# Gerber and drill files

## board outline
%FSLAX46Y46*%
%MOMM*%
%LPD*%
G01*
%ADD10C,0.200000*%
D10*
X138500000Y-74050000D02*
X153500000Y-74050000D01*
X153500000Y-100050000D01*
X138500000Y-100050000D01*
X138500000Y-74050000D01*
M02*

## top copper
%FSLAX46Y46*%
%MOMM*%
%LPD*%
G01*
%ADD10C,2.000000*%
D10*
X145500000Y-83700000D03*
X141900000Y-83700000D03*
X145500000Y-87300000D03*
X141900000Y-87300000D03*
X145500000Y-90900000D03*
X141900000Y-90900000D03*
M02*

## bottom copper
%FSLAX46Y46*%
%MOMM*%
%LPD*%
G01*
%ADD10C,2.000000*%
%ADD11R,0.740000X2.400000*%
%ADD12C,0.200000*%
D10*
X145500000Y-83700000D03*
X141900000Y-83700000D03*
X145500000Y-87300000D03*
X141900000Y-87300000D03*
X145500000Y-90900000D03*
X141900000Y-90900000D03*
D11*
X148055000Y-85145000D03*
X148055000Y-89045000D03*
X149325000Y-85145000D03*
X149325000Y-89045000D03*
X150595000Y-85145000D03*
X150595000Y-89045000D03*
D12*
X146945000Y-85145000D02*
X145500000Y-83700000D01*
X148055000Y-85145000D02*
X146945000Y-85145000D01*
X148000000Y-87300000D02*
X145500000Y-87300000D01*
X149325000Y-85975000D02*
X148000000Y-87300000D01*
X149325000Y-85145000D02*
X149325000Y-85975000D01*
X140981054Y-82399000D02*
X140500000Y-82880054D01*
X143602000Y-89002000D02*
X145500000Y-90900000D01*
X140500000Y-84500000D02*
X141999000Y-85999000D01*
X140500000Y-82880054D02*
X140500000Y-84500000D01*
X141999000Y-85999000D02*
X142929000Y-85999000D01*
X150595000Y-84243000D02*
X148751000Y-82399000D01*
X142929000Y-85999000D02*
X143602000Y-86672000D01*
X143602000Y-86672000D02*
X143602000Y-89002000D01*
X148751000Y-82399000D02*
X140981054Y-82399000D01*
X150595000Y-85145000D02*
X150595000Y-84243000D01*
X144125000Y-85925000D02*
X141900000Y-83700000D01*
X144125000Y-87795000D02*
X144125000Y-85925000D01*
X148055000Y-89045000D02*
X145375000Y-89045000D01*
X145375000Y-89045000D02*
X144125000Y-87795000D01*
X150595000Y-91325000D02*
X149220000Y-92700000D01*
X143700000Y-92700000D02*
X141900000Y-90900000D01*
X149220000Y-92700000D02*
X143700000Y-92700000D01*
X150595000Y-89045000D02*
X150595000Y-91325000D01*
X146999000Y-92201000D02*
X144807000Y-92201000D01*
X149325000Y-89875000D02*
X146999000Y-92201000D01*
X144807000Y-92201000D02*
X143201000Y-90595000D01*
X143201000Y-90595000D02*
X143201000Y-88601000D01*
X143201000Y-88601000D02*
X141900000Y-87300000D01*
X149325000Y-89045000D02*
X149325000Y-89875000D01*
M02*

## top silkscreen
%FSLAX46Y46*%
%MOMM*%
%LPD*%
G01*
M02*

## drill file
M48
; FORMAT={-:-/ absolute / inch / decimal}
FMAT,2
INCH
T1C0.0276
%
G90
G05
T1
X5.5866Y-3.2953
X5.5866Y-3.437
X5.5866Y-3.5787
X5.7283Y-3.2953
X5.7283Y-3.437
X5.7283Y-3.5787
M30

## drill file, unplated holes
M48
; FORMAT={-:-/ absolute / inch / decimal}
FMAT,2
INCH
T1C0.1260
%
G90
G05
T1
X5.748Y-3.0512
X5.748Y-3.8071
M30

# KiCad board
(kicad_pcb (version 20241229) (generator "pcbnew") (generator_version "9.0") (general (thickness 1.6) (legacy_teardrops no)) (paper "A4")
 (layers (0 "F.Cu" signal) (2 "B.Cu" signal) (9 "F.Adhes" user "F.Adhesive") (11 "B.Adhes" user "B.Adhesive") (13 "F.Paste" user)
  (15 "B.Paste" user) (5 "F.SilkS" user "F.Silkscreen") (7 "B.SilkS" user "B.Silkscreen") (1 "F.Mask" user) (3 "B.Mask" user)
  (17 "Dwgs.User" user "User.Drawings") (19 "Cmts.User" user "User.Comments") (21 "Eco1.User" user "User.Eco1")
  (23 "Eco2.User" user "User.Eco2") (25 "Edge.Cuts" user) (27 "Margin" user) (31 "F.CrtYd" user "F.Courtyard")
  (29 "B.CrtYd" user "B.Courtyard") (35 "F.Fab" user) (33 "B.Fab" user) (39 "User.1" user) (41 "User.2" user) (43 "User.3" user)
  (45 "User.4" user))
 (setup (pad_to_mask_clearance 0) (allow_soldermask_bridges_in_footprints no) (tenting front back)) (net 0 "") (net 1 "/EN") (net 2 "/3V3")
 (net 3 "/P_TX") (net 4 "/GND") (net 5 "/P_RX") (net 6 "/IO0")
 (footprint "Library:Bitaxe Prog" (layer "F.Cu") (at 141.9 83.7)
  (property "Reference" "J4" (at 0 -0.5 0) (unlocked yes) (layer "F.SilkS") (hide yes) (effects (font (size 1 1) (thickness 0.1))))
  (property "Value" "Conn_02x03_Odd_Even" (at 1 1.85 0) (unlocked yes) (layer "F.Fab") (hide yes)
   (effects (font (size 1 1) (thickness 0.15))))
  (pad "1" thru_hole circle (at 3.6 0) (size 2 2) (drill 0.7) (layers "*.Cu" "F.Mask") (remove_unused_layers no) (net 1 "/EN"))
  (pad "2" thru_hole circle (at 0 0) (size 2 2) (drill 0.7) (layers "*.Cu" "F.Mask") (remove_unused_layers no) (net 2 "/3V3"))
  (pad "3" thru_hole circle (at 3.6 3.6 90) (size 2 2) (drill 0.7) (layers "*.Cu" "F.Mask") (remove_unused_layers no) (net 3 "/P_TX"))
  (pad "4" thru_hole circle (at 0 3.6) (size 2 2) (drill 0.7) (layers "*.Cu" "F.Mask") (remove_unused_layers no) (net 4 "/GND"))
  (pad "5" thru_hole circle (at 3.6 7.2) (size 2 2) (drill 0.7) (layers "*.Cu" "F.Mask") (remove_unused_layers no) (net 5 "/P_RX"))
  (pad "6" thru_hole circle (at 0 7.2) (size 2 2) (drill 0.7) (layers "*.Cu" "F.Mask") (remove_unused_layers no) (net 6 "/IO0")))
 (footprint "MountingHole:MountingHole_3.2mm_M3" (layer "F.Cu") (at 146 96.7)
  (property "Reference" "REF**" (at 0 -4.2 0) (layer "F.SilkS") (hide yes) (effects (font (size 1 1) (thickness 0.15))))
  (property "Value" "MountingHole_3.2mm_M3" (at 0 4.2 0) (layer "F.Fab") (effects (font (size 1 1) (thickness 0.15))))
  (pad "" np_thru_hole circle (at 0 0) (size 3.2 3.2) (drill 3.2) (layers "*.Cu" "*.Mask")))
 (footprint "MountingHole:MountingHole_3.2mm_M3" (layer "F.Cu") (at 146 77.5)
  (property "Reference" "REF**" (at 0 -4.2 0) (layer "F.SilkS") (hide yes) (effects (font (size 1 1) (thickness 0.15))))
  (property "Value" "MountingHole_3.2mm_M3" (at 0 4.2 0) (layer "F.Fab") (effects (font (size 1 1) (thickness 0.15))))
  (pad "" np_thru_hole circle (at 0 0) (size 3.2 3.2) (drill 3.2) (layers "*.Cu" "*.Mask")))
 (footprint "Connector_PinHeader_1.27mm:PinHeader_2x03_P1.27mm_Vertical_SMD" (layer "B.Cu") (at 149.325 87.095 -90)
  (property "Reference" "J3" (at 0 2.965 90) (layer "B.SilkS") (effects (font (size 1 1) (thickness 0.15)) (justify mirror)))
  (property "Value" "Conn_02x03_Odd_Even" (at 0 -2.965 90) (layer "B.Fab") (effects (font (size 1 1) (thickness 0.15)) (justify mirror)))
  (pad "1" smd rect (at -1.95 1.27 270) (size 2.4 0.74) (layers "B.Cu" "B.Mask" "B.Paste") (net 1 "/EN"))
  (pad "2" smd rect (at 1.95 1.27 270) (size 2.4 0.74) (layers "B.Cu" "B.Mask" "B.Paste") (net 2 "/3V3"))
  (pad "3" smd rect (at -1.95 0 270) (size 2.4 0.74) (layers "B.Cu" "B.Mask" "B.Paste") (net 3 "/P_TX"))
  (pad "4" smd rect (at 1.95 0 270) (size 2.4 0.74) (layers "B.Cu" "B.Mask" "B.Paste") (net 4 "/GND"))
  (pad "5" smd rect (at -1.95 -1.27 270) (size 2.4 0.74) (layers "B.Cu" "B.Mask" "B.Paste") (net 5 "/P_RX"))
  (pad "6" smd rect (at 1.95 -1.27 270) (size 2.4 0.74) (layers "B.Cu" "B.Mask" "B.Paste") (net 6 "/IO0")))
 (gr_rect (start 138.5 74.05) (end 153.5 100.05) (stroke (width 0.2) (type solid)) (fill no) (layer "Edge.Cuts"))
 (segment (start 146.945 85.145) (end 145.5 83.7) (width 0.2) (layer "B.Cu") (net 1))
 (segment (start 148.055 85.145) (end 146.945 85.145) (width 0.2) (layer "B.Cu") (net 1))
 (segment (start 148 87.3) (end 145.5 87.3) (width 0.2) (layer "B.Cu") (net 3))
 (segment (start 149.325 85.975) (end 148 87.3) (width 0.2) (layer "B.Cu") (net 3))
 (segment (start 149.325 85.145) (end 149.325 85.975) (width 0.2) (layer "B.Cu") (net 3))
 (segment (start 140.981054 82.399) (end 140.5 82.880054) (width 0.2) (layer "B.Cu") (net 5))
 (segment (start 143.602 89.002) (end 145.5 90.9) (width 0.2) (layer "B.Cu") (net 5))
 (segment (start 140.5 84.5) (end 141.999 85.999) (width 0.2) (layer "B.Cu") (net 5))
 (segment (start 140.5 82.880054) (end 140.5 84.5) (width 0.2) (layer "B.Cu") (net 5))
 (segment (start 141.999 85.999) (end 142.929 85.999) (width 0.2) (layer "B.Cu") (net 5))
 (segment (start 150.595 84.243) (end 148.751 82.399) (width 0.2) (layer "B.Cu") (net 5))
 (segment (start 142.929 85.999) (end 143.602 86.672) (width 0.2) (layer "B.Cu") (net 5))
 (segment (start 143.602 86.672) (end 143.602 89.002) (width 0.2) (layer "B.Cu") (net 5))
 (segment (start 148.751 82.399) (end 140.981054 82.399) (width 0.2) (layer "B.Cu") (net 5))
 (segment (start 150.595 85.145) (end 150.595 84.243) (width 0.2) (layer "B.Cu") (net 5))
 (segment (start 144.125 85.925) (end 141.9 83.7) (width 0.2) (layer "B.Cu") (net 2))
 (segment (start 144.125 87.795) (end 144.125 85.925) (width 0.2) (layer "B.Cu") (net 2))
 (segment (start 148.055 89.045) (end 145.375 89.045) (width 0.2) (layer "B.Cu") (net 2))
 (segment (start 145.375 89.045) (end 144.125 87.795) (width 0.2) (layer "B.Cu") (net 2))
 (segment (start 150.595 91.325) (end 149.22 92.7) (width 0.2) (layer "B.Cu") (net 6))
 (segment (start 143.7 92.7) (end 141.9 90.9) (width 0.2) (layer "B.Cu") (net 6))
 (segment (start 149.22 92.7) (end 143.7 92.7) (width 0.2) (layer "B.Cu") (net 6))
 (segment (start 150.595 89.045) (end 150.595 91.325) (width 0.2) (layer "B.Cu") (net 6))
 (segment (start 146.999 92.201) (end 144.807 92.201) (width 0.2) (layer "B.Cu") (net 4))
 (segment (start 149.325 89.875) (end 146.999 92.201) (width 0.2) (layer "B.Cu") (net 4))
 (segment (start 144.807 92.201) (end 143.201 90.595) (width 0.2) (layer "B.Cu") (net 4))
 (segment (start 143.201 90.595) (end 143.201 88.601) (width 0.2) (layer "B.Cu") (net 4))
 (segment (start 143.201 88.601) (end 141.9 87.3) (width 0.2) (layer "B.Cu") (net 4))
 (segment (start 149.325 89.045) (end 149.325 89.875) (width 0.2) (layer "B.Cu") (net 4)))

